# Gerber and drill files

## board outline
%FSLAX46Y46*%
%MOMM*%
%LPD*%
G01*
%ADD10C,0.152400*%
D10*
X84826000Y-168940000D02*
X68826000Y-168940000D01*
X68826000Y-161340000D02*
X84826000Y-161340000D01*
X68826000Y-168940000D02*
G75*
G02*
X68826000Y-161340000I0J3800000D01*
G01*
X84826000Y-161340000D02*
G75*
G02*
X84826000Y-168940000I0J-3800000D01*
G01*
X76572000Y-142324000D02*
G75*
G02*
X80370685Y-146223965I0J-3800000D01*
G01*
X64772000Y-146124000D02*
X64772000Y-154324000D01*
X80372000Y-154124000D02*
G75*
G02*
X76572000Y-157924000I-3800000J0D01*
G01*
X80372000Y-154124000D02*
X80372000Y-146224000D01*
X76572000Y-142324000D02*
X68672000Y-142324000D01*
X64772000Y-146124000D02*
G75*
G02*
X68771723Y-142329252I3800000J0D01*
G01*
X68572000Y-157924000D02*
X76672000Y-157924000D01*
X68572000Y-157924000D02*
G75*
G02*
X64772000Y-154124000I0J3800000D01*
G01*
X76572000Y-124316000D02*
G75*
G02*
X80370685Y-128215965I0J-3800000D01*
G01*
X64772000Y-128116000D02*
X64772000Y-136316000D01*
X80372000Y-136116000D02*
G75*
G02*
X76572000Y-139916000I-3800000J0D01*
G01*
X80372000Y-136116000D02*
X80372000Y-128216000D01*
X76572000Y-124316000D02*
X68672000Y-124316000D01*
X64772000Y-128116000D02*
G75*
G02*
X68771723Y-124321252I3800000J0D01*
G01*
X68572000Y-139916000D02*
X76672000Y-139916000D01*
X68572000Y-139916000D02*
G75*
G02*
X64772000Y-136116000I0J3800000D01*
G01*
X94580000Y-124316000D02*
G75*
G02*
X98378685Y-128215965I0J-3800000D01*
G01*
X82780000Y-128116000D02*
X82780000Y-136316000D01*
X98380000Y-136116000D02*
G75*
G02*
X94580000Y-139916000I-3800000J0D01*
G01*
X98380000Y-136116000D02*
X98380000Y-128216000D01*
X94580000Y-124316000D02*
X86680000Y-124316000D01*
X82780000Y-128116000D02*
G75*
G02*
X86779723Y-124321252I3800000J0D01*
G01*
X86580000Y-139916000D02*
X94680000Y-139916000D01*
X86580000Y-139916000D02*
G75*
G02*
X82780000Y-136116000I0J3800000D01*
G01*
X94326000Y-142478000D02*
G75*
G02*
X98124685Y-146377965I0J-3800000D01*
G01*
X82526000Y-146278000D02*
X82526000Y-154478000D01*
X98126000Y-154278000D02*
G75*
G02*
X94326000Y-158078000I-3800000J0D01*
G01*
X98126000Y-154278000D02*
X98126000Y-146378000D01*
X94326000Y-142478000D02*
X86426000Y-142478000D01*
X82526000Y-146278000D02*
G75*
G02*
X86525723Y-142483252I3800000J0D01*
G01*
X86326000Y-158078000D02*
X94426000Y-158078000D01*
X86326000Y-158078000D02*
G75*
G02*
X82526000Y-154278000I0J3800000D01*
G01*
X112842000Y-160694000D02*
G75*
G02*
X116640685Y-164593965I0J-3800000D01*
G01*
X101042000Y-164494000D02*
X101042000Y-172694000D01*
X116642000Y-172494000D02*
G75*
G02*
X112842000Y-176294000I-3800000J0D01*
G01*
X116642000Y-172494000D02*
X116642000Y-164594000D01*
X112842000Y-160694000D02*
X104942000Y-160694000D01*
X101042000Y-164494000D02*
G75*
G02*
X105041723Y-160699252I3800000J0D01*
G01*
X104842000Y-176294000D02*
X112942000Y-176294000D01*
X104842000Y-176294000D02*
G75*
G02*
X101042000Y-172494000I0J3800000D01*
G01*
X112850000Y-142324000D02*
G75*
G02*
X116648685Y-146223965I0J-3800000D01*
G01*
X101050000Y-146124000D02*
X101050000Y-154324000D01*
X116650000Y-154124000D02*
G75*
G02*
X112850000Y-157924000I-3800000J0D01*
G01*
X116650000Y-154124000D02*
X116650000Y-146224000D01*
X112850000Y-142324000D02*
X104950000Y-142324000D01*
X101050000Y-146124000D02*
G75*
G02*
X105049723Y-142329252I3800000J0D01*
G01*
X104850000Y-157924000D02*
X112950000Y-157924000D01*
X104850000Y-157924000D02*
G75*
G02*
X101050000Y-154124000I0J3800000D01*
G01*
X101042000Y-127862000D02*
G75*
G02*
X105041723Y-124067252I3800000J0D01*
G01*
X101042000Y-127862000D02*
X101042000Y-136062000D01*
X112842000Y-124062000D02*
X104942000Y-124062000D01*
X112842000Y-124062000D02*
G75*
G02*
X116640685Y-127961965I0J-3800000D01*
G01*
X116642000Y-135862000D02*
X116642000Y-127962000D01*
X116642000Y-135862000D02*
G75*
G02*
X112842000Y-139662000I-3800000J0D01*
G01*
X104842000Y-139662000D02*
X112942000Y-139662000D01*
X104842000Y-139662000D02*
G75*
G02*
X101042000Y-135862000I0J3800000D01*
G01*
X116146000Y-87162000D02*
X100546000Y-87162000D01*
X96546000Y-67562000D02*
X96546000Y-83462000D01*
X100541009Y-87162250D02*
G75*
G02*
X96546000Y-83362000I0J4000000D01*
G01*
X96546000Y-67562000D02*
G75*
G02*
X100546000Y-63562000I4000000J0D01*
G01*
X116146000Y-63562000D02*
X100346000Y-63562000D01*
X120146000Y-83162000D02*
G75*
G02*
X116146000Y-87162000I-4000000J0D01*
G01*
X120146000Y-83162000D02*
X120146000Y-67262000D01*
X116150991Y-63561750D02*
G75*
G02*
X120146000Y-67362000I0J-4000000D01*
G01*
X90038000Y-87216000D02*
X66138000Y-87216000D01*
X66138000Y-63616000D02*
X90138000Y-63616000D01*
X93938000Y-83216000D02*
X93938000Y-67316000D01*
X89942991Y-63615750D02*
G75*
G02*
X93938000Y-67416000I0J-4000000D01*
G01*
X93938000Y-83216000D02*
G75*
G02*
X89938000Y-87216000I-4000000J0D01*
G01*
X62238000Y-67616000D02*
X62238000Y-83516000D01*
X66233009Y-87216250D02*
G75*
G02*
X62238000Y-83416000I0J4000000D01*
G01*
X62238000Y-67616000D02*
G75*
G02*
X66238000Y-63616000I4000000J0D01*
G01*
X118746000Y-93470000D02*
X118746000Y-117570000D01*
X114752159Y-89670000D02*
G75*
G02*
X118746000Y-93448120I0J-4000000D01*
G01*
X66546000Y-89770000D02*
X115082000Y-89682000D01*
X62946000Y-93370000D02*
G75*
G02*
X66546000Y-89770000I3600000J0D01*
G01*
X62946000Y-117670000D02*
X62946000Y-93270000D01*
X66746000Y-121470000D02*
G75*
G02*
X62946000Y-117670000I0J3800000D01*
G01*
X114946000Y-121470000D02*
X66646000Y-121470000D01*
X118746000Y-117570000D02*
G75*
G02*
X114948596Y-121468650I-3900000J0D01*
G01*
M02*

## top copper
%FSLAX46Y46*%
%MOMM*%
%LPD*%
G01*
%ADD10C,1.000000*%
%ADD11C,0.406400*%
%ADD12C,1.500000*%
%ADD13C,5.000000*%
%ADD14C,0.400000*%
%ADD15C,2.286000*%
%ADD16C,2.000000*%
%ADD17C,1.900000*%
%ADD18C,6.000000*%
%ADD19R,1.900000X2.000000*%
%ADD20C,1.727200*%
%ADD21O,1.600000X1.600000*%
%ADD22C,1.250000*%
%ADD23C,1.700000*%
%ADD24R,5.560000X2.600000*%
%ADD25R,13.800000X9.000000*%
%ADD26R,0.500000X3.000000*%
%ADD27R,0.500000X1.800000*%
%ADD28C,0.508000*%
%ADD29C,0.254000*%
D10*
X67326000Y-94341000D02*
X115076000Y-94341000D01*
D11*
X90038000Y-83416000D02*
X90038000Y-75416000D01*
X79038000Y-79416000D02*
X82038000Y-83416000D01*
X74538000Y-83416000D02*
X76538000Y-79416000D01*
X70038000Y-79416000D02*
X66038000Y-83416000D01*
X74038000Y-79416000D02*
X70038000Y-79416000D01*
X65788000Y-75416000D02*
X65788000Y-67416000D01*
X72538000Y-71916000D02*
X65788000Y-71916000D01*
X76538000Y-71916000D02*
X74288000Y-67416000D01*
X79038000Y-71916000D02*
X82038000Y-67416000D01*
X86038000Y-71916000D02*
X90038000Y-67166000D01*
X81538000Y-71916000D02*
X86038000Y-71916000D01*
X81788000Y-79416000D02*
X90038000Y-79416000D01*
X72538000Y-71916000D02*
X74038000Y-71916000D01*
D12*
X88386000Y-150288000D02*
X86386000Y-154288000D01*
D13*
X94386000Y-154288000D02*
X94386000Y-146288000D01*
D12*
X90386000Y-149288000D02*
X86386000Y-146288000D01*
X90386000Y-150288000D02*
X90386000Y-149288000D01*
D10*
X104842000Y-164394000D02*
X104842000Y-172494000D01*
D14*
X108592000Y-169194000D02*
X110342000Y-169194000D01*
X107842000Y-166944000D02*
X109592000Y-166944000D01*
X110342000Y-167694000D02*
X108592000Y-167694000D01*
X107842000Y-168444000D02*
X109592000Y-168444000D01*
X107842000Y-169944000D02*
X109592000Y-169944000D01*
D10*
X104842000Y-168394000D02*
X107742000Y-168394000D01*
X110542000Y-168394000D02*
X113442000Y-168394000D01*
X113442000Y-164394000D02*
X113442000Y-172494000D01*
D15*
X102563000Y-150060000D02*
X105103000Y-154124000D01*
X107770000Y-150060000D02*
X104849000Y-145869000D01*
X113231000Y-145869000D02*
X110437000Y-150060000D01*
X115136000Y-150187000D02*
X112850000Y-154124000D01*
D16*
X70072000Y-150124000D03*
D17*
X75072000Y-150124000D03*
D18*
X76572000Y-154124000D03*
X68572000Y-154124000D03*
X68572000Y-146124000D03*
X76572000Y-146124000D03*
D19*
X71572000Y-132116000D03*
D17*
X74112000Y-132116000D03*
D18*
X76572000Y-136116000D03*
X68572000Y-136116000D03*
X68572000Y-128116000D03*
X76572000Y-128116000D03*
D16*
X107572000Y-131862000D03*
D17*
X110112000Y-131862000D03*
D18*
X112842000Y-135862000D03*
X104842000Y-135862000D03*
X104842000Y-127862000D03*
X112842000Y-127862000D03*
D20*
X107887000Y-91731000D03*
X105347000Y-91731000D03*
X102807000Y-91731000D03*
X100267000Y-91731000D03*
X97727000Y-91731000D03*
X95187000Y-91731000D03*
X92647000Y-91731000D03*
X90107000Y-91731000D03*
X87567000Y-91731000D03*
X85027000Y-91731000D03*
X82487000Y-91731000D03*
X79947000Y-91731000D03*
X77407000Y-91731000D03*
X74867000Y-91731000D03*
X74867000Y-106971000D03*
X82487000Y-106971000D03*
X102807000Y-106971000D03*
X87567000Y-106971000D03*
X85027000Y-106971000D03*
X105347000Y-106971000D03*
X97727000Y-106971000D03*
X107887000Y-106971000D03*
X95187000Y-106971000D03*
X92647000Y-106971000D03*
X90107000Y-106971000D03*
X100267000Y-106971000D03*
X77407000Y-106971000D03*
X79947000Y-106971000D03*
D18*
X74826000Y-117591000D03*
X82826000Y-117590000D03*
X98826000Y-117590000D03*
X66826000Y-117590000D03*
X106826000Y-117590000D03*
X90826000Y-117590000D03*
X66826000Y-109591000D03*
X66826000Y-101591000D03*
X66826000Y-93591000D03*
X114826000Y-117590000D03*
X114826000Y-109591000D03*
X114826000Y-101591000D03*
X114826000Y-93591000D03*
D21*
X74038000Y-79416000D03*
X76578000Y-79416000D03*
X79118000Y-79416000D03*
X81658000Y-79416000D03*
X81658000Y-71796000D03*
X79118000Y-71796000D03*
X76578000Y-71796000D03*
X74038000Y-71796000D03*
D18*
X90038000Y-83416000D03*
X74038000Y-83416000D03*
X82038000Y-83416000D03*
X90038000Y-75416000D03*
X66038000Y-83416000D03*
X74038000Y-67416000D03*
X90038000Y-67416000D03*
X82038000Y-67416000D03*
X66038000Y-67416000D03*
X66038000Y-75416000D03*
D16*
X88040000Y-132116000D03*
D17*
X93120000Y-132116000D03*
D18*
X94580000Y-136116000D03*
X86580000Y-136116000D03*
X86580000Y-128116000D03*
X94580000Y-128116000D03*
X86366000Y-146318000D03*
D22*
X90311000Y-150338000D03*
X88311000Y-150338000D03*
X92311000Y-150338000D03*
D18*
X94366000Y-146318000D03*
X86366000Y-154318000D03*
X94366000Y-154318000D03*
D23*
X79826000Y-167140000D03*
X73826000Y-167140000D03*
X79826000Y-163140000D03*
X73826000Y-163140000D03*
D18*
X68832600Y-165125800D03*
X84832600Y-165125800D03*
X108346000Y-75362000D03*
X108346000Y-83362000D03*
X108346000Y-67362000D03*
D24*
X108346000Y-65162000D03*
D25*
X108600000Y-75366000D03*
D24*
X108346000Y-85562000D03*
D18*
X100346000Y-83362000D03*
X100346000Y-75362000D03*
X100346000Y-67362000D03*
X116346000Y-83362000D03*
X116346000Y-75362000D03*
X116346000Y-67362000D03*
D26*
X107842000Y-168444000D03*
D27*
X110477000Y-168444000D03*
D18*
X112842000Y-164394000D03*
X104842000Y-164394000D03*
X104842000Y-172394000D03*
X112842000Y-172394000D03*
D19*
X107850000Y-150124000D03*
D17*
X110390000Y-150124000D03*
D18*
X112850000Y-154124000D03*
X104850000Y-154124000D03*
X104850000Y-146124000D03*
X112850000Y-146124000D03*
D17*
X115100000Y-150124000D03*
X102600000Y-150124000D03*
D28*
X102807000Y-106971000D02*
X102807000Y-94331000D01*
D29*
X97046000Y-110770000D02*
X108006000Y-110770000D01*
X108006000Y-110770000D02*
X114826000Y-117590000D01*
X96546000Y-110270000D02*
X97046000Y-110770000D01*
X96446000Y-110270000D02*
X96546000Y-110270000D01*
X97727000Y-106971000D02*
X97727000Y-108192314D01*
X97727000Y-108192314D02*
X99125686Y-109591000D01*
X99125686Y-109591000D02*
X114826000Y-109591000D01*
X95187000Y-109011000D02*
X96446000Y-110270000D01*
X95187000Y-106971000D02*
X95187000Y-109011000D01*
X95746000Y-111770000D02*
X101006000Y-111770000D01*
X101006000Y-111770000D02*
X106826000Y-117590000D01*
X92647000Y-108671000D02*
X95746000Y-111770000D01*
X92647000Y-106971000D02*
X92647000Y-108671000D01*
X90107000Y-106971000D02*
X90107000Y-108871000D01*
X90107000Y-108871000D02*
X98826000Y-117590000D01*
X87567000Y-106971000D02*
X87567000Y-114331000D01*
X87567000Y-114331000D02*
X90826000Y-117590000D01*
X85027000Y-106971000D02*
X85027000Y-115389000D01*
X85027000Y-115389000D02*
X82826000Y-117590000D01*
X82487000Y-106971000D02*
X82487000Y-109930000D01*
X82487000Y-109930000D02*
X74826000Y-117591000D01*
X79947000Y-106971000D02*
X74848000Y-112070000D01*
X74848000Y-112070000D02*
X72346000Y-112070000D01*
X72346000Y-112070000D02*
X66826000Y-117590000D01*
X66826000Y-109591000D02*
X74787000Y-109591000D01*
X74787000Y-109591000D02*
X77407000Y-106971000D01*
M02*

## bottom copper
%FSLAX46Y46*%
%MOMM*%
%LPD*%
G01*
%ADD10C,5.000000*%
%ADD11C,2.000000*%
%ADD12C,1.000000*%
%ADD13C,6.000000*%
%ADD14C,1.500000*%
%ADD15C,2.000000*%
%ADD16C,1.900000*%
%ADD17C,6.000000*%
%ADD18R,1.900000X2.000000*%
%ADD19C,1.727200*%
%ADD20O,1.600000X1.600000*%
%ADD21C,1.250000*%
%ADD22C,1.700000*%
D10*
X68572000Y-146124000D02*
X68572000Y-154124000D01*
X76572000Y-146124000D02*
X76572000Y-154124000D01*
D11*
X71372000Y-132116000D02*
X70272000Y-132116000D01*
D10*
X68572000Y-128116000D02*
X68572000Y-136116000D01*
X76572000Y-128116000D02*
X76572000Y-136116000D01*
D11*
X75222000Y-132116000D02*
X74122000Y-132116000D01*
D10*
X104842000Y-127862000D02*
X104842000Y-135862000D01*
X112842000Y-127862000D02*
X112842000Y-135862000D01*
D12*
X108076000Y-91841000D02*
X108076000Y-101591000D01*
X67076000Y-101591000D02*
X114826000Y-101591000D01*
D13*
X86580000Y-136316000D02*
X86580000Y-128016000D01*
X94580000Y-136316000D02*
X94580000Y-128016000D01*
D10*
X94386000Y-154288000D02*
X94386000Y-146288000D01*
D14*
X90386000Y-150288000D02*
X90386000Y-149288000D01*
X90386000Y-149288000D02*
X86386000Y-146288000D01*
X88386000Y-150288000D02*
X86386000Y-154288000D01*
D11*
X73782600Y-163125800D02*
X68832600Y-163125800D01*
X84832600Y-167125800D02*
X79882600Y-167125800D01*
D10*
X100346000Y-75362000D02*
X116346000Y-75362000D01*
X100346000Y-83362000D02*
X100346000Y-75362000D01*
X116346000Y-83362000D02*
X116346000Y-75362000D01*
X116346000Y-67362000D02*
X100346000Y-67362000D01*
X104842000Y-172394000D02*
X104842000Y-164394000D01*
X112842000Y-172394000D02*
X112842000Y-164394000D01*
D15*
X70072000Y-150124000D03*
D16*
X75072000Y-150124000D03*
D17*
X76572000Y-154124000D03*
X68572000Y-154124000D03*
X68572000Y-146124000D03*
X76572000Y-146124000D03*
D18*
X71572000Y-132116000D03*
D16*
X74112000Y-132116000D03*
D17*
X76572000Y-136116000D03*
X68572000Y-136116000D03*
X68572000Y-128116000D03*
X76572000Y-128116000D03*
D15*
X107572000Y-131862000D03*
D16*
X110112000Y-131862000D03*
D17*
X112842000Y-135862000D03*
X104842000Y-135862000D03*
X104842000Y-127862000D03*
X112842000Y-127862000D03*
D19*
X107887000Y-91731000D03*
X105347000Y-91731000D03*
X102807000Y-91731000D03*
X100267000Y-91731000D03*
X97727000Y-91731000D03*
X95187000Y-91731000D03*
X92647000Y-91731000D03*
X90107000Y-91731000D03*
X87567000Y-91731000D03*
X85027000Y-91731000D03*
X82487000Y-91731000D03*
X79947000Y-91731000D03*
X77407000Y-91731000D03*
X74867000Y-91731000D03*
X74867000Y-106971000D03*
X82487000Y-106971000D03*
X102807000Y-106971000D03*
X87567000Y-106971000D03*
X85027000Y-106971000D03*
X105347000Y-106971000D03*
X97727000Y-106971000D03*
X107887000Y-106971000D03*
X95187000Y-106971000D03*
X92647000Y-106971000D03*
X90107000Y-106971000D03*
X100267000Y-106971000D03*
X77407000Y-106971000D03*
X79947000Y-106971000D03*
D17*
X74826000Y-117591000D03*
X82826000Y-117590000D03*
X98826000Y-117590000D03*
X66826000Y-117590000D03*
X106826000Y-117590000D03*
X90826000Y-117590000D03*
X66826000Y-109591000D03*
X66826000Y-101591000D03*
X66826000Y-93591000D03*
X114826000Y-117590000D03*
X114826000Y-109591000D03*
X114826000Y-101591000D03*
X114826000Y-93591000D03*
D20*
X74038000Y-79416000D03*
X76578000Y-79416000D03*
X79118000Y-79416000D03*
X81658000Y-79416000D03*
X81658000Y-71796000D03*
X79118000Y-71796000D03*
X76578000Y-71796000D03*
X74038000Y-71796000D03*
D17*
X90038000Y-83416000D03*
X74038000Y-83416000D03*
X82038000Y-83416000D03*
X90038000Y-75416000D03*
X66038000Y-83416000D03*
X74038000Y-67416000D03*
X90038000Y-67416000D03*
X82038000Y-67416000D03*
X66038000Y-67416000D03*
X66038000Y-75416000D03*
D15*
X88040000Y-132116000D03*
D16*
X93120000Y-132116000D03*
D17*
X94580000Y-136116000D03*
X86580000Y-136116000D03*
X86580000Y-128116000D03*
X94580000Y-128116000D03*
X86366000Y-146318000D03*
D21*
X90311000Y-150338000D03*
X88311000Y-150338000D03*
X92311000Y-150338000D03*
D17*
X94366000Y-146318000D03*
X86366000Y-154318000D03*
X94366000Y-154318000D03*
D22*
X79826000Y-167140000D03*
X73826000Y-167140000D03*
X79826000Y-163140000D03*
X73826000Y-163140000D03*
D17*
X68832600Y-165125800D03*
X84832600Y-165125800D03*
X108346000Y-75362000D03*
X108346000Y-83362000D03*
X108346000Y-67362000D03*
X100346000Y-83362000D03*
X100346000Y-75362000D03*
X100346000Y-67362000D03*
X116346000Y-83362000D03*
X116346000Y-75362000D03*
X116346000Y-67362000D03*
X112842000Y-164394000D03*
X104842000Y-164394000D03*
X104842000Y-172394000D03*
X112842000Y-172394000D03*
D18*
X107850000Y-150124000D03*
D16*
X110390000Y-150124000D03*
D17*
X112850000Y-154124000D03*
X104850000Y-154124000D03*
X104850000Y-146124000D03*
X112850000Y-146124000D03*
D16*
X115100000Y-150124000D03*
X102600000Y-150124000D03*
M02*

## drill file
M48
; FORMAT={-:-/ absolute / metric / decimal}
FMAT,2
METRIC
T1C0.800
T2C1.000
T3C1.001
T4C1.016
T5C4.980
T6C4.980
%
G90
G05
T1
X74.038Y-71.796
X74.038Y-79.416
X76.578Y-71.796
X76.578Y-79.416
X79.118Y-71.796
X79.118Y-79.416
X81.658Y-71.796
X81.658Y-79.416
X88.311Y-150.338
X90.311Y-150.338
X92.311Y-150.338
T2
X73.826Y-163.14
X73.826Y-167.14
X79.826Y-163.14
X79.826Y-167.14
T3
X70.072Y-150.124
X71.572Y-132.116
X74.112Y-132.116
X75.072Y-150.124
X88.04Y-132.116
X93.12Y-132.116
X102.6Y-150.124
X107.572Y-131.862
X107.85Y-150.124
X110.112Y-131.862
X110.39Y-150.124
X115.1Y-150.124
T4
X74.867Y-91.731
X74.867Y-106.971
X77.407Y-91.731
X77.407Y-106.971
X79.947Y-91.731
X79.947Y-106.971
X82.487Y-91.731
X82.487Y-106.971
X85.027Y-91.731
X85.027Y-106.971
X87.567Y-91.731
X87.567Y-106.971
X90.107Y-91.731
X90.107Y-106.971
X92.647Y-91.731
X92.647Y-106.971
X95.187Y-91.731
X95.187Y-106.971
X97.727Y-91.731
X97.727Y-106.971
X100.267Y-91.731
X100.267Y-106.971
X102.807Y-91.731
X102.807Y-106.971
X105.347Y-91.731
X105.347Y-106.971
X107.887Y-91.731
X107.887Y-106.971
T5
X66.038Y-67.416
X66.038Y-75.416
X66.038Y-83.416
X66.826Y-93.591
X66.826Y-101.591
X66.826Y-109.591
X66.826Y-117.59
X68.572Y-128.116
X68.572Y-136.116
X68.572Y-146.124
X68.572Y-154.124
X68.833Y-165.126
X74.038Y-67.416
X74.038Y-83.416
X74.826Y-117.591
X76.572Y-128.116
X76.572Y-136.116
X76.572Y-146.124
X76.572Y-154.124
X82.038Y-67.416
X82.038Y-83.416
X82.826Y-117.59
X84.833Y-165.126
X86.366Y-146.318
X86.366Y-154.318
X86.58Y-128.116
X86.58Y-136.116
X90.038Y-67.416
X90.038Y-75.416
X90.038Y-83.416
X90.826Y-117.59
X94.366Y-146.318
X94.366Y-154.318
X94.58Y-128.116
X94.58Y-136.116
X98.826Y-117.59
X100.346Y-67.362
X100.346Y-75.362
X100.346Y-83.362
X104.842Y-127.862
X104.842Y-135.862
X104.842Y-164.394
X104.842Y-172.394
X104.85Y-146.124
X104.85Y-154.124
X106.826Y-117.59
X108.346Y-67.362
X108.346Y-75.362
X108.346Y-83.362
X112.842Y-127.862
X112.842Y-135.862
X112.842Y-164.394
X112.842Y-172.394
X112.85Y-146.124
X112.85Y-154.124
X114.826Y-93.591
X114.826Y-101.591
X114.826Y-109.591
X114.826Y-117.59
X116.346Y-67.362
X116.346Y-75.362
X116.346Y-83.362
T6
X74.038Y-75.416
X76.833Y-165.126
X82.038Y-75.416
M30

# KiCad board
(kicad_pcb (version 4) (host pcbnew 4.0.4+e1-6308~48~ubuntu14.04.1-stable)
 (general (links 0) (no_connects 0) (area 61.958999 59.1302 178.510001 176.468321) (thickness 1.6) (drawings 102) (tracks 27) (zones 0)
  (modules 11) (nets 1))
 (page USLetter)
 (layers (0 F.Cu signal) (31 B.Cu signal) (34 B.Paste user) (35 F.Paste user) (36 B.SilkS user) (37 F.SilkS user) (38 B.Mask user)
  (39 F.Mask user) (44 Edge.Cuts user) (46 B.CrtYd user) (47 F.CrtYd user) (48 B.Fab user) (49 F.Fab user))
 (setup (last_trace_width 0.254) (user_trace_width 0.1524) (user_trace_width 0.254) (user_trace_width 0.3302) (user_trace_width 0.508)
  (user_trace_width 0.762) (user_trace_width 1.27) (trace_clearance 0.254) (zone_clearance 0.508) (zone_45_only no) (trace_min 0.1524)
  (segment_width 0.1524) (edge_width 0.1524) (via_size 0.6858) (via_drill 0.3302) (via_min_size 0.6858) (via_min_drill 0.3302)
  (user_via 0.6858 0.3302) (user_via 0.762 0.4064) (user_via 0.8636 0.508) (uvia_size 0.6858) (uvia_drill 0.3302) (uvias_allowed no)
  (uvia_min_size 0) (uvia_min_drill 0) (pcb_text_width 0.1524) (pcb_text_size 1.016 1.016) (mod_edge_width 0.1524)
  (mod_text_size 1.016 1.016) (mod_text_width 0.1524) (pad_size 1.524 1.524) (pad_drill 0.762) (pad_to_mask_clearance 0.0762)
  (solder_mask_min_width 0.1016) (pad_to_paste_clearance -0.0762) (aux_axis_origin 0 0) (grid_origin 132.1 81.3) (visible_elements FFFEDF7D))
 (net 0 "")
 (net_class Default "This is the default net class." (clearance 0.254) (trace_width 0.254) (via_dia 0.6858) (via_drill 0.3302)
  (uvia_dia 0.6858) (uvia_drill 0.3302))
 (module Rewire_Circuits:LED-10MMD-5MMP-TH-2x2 (layer F.Cu) (at 76.572 154.124 90)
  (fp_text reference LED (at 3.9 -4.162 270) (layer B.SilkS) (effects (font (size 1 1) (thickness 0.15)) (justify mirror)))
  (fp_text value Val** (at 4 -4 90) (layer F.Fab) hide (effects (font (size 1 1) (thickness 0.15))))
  (fp_line (start 8 -8) (end 0 -8) (layer B.Cu) (width 5)) (fp_line (start 8 0) (end 0 0) (layer B.Cu) (width 5))
  (pad + thru_hole circle (at 4 -6.5 90) (size 2 2) (drill 1.00076) (layers *.Cu *.Mask F.SilkS))
  (pad - thru_hole circle (at 4 -1.5) (size 1.9 1.9) (drill 1.00076) (layers *.Cu *.Mask F.SilkS))
  (pad - thru_hole circle (at 0 0 90) (size 6 6) (drill 4.98) (layers *.Cu *.Mask))
  (pad + thru_hole circle (at 0 -8 90) (size 6 6) (drill 4.98) (layers *.Cu *.Mask))
  (pad + thru_hole circle (at 8 -8 90) (size 6 6) (drill 4.98) (layers *.Cu *.Mask))
  (pad - thru_hole circle (at 8 0 90) (size 6 6) (drill 4.98) (layers *.Cu *.Mask)))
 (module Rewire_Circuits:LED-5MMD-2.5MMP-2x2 (layer F.Cu) (at 76.572 136.116 90)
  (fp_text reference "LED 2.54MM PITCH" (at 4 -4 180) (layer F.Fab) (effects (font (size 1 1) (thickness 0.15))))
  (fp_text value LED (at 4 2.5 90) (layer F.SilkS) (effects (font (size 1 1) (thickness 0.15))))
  (fp_line (start 4 -5.2) (end 4 -6.3) (layer B.Cu) (width 2)) (fp_line (start 8 -8) (end 0 -8) (layer B.Cu) (width 5))
  (fp_line (start 8 0) (end 0 0) (layer B.Cu) (width 5))
  (fp_line (start 4 -1.35) (end 4 -2.45) (layer B.Cu) (width 2))
  (pad - thru_hole rect (at 4 -5 90) (size 2 1.9) (drill 1.00076) (layers *.Cu *.Mask))
  (pad + thru_hole circle (at 4 -2.46) (size 1.9 1.9) (drill 1.00076) (layers *.Cu *.Mask))
  (pad + thru_hole circle (at 0 0 90) (size 6 6) (drill 4.98) (layers *.Cu *.Mask))
  (pad - thru_hole circle (at 0 -8 90) (size 6 6) (drill 4.98) (layers *.Cu *.Mask))
  (pad - thru_hole circle (at 8 -8 90) (size 6 6) (drill 4.98) (layers *.Cu *.Mask))
  (pad + thru_hole circle (at 8 0 90) (size 6 6) (drill 4.98) (layers *.Cu *.Mask)))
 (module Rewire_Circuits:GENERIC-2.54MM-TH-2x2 (layer F.Cu) (at 112.842 135.862 90)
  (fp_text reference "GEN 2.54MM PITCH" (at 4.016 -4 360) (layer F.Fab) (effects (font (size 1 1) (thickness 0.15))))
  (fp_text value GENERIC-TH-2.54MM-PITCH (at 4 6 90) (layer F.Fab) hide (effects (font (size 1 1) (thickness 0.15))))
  (fp_line (start 8 -8) (end 0 -8) (layer B.Cu) (width 5)) (fp_line (start 8 0) (end 0 0) (layer B.Cu) (width 5))
  (pad 1 thru_hole circle (at 4 -5.27 90) (size 2 2) (drill 1.00076) (layers *.Cu *.Mask F.SilkS))
  (pad 2 thru_hole circle (at 4 -2.73) (size 1.9 1.9) (drill 1.00076) (layers *.Cu *.Mask F.SilkS))
  (pad 2 thru_hole circle (at 0 0 90) (size 6 6) (drill 4.98) (layers *.Cu *.Mask))
  (pad 1 thru_hole circle (at 0 -8 90) (size 6 6) (drill 4.98) (layers *.Cu *.Mask))
  (pad 1 thru_hole circle (at 8 -8 90) (size 6 6) (drill 4.98) (layers *.Cu *.Mask))
  (pad 2 thru_hole circle (at 8 0 90) (size 6 6) (drill 4.98) (layers *.Cu *.Mask)))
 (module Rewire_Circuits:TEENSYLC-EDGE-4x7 (layer F.Cu) (at 66.826 117.591 90)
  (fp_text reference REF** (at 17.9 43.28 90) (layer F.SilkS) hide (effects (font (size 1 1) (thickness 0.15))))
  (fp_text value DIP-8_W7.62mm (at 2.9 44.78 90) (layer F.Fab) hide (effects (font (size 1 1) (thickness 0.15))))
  (fp_line (start 25.75 41.25) (end 16 41.25) (layer B.Cu) (width 1)) (fp_line (start 16 0.25) (end 16 48) (layer B.Cu) (width 1))
  (fp_line (start 23.25 0.5) (end 23.25 48.25) (layer F.Cu) (width 1))
  (pad GND thru_hole circle (at 25.86 41.061 270) (size 1.7272 1.7272) (drill 1.016) (layers *.Cu *.Mask F.SilkS))
  (pad 0 thru_hole circle (at 25.86 38.521 270) (size 1.7272 1.7272) (drill 1.016) (layers *.Cu *.Mask F.SilkS))
  (pad 1 thru_hole circle (at 25.86 35.981 270) (size 1.7272 1.7272) (drill 1.016) (layers *.Cu *.Mask F.SilkS))
  (pad 2 thru_hole circle (at 25.86 33.441 270) (size 1.7272 1.7272) (drill 1.016) (layers *.Cu *.Mask F.SilkS))
  (pad 3 thru_hole circle (at 25.86 30.901 270) (size 1.7272 1.7272) (drill 1.016) (layers *.Cu *.Mask F.SilkS))
  (pad 4 thru_hole circle (at 25.86 28.361 270) (size 1.7272 1.7272) (drill 1.016) (layers *.Cu *.Mask F.SilkS))
  (pad 5 thru_hole circle (at 25.86 25.821 270) (size 1.7272 1.7272) (drill 1.016) (layers *.Cu *.Mask F.SilkS))
  (pad 6 thru_hole circle (at 25.86 23.281 270) (size 1.7272 1.7272) (drill 1.016) (layers *.Cu *.Mask F.SilkS))
  (pad 7 thru_hole circle (at 25.86 20.741 270) (size 1.7272 1.7272) (drill 1.016) (layers *.Cu *.Mask F.SilkS))
  (pad 8 thru_hole circle (at 25.86 18.201 270) (size 1.7272 1.7272) (drill 1.016) (layers *.Cu *.Mask F.SilkS))
  (pad 9 thru_hole circle (at 25.86 15.661 270) (size 1.7272 1.7272) (drill 1.016) (layers *.Cu *.Mask F.SilkS))
  (pad 10 thru_hole circle (at 25.86 13.121 270) (size 1.7272 1.7272) (drill 1.016) (layers *.Cu *.Mask F.SilkS))
  (pad 11 thru_hole circle (at 25.86 10.581 270) (size 1.7272 1.7272) (drill 1.016) (layers *.Cu *.Mask F.SilkS))
  (pad 12 thru_hole circle (at 25.86 8.041 270) (size 1.7272 1.7272) (drill 1.016) (layers *.Cu *.Mask F.SilkS))
  (pad 13 thru_hole circle (at 10.62 8.041 270) (size 1.7272 1.7272) (drill 1.016) (layers *.Cu *.Mask F.SilkS))
  (pad 16 thru_hole circle (at 10.62 15.661 270) (size 1.7272 1.7272) (drill 1.016) (layers *.Cu *.Mask F.SilkS))
  (pad 3.3V thru_hole circle (at 10.62 35.981 270) (size 1.7272 1.7272) (drill 1.016) (layers *.Cu *.Mask F.SilkS))
  (pad 18 thru_hole circle (at 10.62 20.741 270) (size 1.7272 1.7272) (drill 1.016) (layers *.Cu *.Mask F.SilkS))
  (pad 17 thru_hole circle (at 10.62 18.201 270) (size 1.7272 1.7272) (drill 1.016) (layers *.Cu *.Mask F.SilkS))
  (pad G3 thru_hole circle (at 10.62 38.521 270) (size 1.7272 1.7272) (drill 1.016) (layers *.Cu *.Mask F.SilkS))
  (pad 22 thru_hole circle (at 10.62 30.901 270) (size 1.7272 1.7272) (drill 1.016) (layers *.Cu *.Mask F.SilkS))
  (pad VIN thru_hole circle (at 10.62 41.061 270) (size 1.7272 1.7272) (drill 1.016) (layers *.Cu *.Mask F.SilkS))
  (pad 21 thru_hole circle (at 10.62 28.361 270) (size 1.7272 1.7272) (drill 1.016) (layers *.Cu *.Mask F.SilkS))
  (pad 20 thru_hole circle (at 10.62 25.821 270) (size 1.7272 1.7272) (drill 1.016) (layers *.Cu *.Mask F.SilkS))
  (pad 19 thru_hole circle (at 10.62 23.281 270) (size 1.7272 1.7272) (drill 1.016) (layers *.Cu *.Mask F.SilkS))
  (pad 23 thru_hole circle (at 10.62 33.441 270) (size 1.7272 1.7272) (drill 1.016) (layers *.Cu *.Mask F.SilkS))
  (pad 14 thru_hole circle (at 10.62 10.581 270) (size 1.7272 1.7272) (drill 1.016) (layers *.Cu *.Mask F.SilkS))
  (pad 15 thru_hole circle (at 10.62 13.121 270) (size 1.7272 1.7272) (drill 1.016) (layers *.Cu *.Mask F.SilkS))
  (pad 16 thru_hole circle (at 0 8 180) (size 6 6) (drill 4.98) (layers *.Cu *.Mask))
  (pad 17 thru_hole circle (at 0.001 16 180) (size 6 6) (drill 4.98) (layers *.Cu *.Mask))
  (pad 19 thru_hole circle (at 0.001 32 180) (size 6 6) (drill 4.98) (layers *.Cu *.Mask))
  (pad 15 thru_hole circle (at 0.001 0 180) (size 6 6) (drill 4.98) (layers *.Cu *.Mask))
  (pad 20 thru_hole circle (at 0.001 40 180) (size 6 6) (drill 4.98) (layers *.Cu *.Mask))
  (pad 18 thru_hole circle (at 0.001 24 180) (size 6 6) (drill 4.98) (layers *.Cu *.Mask))
  (pad 14 thru_hole circle (at 8 0 180) (size 6 6) (drill 4.98) (layers *.Cu *.Mask))
  (pad GND thru_hole circle (at 16 0 180) (size 6 6) (drill 4.98) (layers *.Cu *.Mask))
  (pad 3.3V thru_hole circle (at 24 0 180) (size 6 6) (drill 4.98) (layers *.Cu *.Mask))
  (pad 21 thru_hole circle (at 0.001 48 180) (size 6 6) (drill 4.98) (layers *.Cu *.Mask))
  (pad 22 thru_hole circle (at 8 48 180) (size 6 6) (drill 4.98) (layers *.Cu *.Mask))
  (pad GND thru_hole circle (at 16 48 180) (size 6 6) (drill 4.98) (layers *.Cu *.Mask))
  (pad 3.3V thru_hole circle (at 24 48 180) (size 6 6) (drill 4.98) (layers *.Cu *.Mask)))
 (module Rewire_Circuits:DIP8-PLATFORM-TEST (layer F.Cu) (at 90.038 83.416 90)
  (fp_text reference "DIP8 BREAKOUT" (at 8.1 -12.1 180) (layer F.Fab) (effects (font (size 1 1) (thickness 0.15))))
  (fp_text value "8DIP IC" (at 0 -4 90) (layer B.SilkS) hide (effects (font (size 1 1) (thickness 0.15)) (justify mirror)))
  (fp_line (start 0 0) (end 8 0) (layer F.Cu) (width 0.4064))
  (fp_line (start 4 -11) (end 0 -8) (layer F.Cu) (width 0.4064))
  (fp_line (start 0 -15.5) (end 4 -13.5) (layer F.Cu) (width 0.4064))
  (fp_line (start 4 -20) (end 0 -24) (layer F.Cu) (width 0.4064))
  (fp_line (start 4 -16) (end 4 -20) (layer F.Cu) (width 0.4064))
  (fp_line (start 8 -24.25) (end 16 -24.25) (layer F.Cu) (width 0.4064))
  (fp_line (start 11.5 -17.5) (end 11.5 -24.25) (layer F.Cu) (width 0.4064))
  (fp_line (start 11.5 -13.5) (end 16 -15.75) (layer F.Cu) (width 0.4064))
  (fp_line (start 11.5 -11) (end 16 -8) (layer F.Cu) (width 0.4064))
  (fp_line (start 11.5 -4) (end 16.25 0) (layer F.Cu) (width 0.4064))
  (fp_line (start 11.5 -8.5) (end 11.5 -4) (layer F.Cu) (width 0.4064))
  (fp_line (start 4 -8.25) (end 4 0) (layer F.Cu) (width 0.4064))
  (fp_line (start 11.5 -17.5) (end 11.5 -16) (layer F.Cu) (width 0.4064))
  (pad 1 thru_hole oval (at 4 -16 90) (size 1.6 1.6) (drill 0.8) (layers *.Cu *.Mask F.SilkS))
  (pad 2 thru_hole oval (at 4 -13.46 90) (size 1.6 1.6) (drill 0.8) (layers *.Cu *.Mask F.SilkS))
  (pad 3 thru_hole oval (at 4 -10.92 90) (size 1.6 1.6) (drill 0.8) (layers *.Cu *.Mask F.SilkS))
  (pad 4 thru_hole oval (at 4 -8.38 90) (size 1.6 1.6) (drill 0.8) (layers *.Cu *.Mask F.SilkS))
  (pad 5 thru_hole oval (at 11.62 -8.38 90) (size 1.6 1.6) (drill 0.8) (layers *.Cu *.Mask F.SilkS))
  (pad 6 thru_hole oval (at 11.62 -10.92 90) (size 1.6 1.6) (drill 0.8) (layers *.Cu *.Mask F.SilkS))
  (pad 7 thru_hole oval (at 11.62 -13.46 90) (size 1.6 1.6) (drill 0.8) (layers *.Cu *.Mask F.SilkS))
  (pad 8 thru_hole oval (at 11.62 -16 90) (size 1.6 1.6) (drill 0.8) (layers *.Cu *.Mask F.SilkS))
  (pad 4 thru_hole circle (at 0 0) (size 6 6) (drill 4.98) (layers *.Cu *.Mask))
  (pad "" np_thru_hole circle (at 8 -16) (size 4.88 4.88) (drill 4.98) (layers *.Cu *.Mask))
  (pad 2 thru_hole circle (at 0 -16) (size 6 6) (drill 4.98) (layers *.Cu *.Mask))
  (pad 3 thru_hole circle (at 0 -8) (size 6 6) (drill 4.98) (layers *.Cu *.Mask))
  (pad "" np_thru_hole circle (at 8 -8) (size 4.88 4.88) (drill 4.98) (layers *.Cu *.Mask F.SilkS))
  (pad 4 thru_hole circle (at 8 0) (size 6 6) (drill 4.98) (layers *.Cu *.Mask))
  (pad 1 thru_hole circle (at 0 -24) (size 6 6) (drill 4.98) (layers *.Cu *.Mask))
  (pad 7 thru_hole circle (at 16 -16) (size 6 6) (drill 4.98) (layers *.Cu *.Mask))
  (pad 5 thru_hole circle (at 16 0) (size 6 6) (drill 4.98) (layers *.Cu *.Mask))
  (pad 6 thru_hole circle (at 16 -8) (size 6 6) (drill 4.98) (layers *.Cu *.Mask))
  (pad 8 thru_hole circle (at 16 -24) (size 6 6) (drill 4.98) (layers *.Cu *.Mask))
  (pad 8 thru_hole circle (at 8 -24) (size 6 6) (drill 4.98) (layers *.Cu *.Mask)))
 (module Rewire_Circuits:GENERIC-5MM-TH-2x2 (layer F.Cu) (at 94.58 136.116 90)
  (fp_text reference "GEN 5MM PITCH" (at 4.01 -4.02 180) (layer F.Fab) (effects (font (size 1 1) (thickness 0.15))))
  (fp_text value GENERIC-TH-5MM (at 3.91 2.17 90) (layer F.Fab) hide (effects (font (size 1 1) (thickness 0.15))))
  (fp_line (start -0.2 -8) (end 8.1 -8) (layer B.Cu) (width 6)) (fp_line (start -0.2 0) (end 8.1 0) (layer B.Cu) (width 6))
  (pad 1 thru_hole circle (at 4 -6.54 90) (size 2 2) (drill 1.00076) (layers *.Cu *.Mask F.SilkS))
  (pad 2 thru_hole circle (at 4 -1.46) (size 1.9 1.9) (drill 1.00076) (layers *.Cu *.Mask F.SilkS))
  (pad 2 thru_hole circle (at 0 0 90) (size 6 6) (drill 4.98) (layers *.Cu *.Mask))
  (pad 1 thru_hole circle (at 0 -8 90) (size 6 6) (drill 4.98) (layers *.Cu *.Mask))
  (pad 1 thru_hole circle (at 8 -8 90) (size 6 6) (drill 4.98) (layers *.Cu *.Mask))
  (pad 2 thru_hole circle (at 8 0 90) (size 6 6) (drill 4.98) (layers *.Cu *.Mask)))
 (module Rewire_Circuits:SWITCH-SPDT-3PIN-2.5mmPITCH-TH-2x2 (layer F.Cu) (at 94.366 154.318 90)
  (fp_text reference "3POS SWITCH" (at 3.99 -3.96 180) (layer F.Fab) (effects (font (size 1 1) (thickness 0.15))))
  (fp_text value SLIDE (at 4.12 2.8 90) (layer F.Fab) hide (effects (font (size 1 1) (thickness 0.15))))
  (fp_line (start 4.03 -5.98) (end 0.03 -7.98) (layer F.Cu) (width 1.5))
  (fp_line (start 0.03 0.02) (end 8.03 0.02) (layer B.Cu) (width 5))
  (fp_line (start 4.03 -3.98) (end 5.03 -3.98) (layer B.Cu) (width 1.5))
  (fp_line (start 5.03 -3.98) (end 8.03 -7.98) (layer B.Cu) (width 1.5))
  (fp_line (start 0.03 0.02) (end 8.03 0.02) (layer F.Cu) (width 5))
  (fp_line (start 5.03 -3.98) (end 8.03 -7.98) (layer F.Cu) (width 1.5))
  (fp_line (start 4.03 -3.98) (end 5.03 -3.98) (layer F.Cu) (width 1.5))
  (fp_line (start 4.03 -5.98) (end 0.03 -7.98) (layer B.Cu) (width 1.5))
  (pad 2 thru_hole circle (at 8 -8 90) (size 6 6) (drill 4.98) (layers *.Cu *.Mask))
  (pad 2 thru_hole circle (at 3.98 -4.055) (size 1.25 1.25) (drill 0.8) (layers *.Cu *.Mask))
  (pad 3 thru_hole circle (at 3.98 -6.055) (size 1.25 1.25) (drill 0.8) (layers *.Cu *.Mask))
  (pad 1 thru_hole circle (at 3.98 -2.055) (size 1.25 1.25) (drill 0.8) (layers *.Cu *.Mask))
  (pad 1 thru_hole circle (at 8 0 90) (size 6 6) (drill 4.98) (layers *.Cu *.Mask))
  (pad 3 thru_hole circle (at 0 -8 90) (size 6 6) (drill 4.98) (layers *.Cu *.Mask))
  (pad 1 thru_hole circle (at 0 0 90) (size 6 6) (drill 4.98) (layers *.Cu *.Mask)))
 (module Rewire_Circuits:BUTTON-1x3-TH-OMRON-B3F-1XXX (layer F.Cu) (at 68.8326 165.1258)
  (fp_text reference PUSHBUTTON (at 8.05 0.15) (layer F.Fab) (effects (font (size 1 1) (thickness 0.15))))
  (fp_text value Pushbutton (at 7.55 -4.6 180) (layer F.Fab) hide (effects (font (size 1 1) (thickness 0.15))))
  (fp_line (start 4.95 -2) (end 0 -2) (layer B.Cu) (width 2)) (fp_line (start 16 2) (end 11.05 2) (layer B.Cu) (width 2))
  (pad 2 thru_hole circle (at 10.9934 2.0142) (size 1.7 1.7) (drill 1) (layers *.Cu *.Mask))
  (pad 2 thru_hole circle (at 4.9934 2.0142) (size 1.7 1.7) (drill 1) (layers *.Cu *.Mask))
  (pad 1 thru_hole circle (at 10.9934 -1.9858) (size 1.7 1.7) (drill 1) (layers *.Cu *.Mask))
  (pad 1 thru_hole circle (at 4.9934 -1.9858) (size 1.7 1.7) (drill 1) (layers *.Cu *.Mask))
  (pad "" np_thru_hole circle (at 8 0) (size 4.88 4.88) (drill 4.98) (layers *.Cu *.Mask F.SilkS))
  (pad 1 thru_hole circle (at 0 0) (size 6 6) (drill 4.98) (layers *.Cu *.Mask F.SilkS))
  (pad 2 thru_hole circle (at 16 0) (size 6 6) (drill 4.98) (layers *.Cu *.Mask F.SilkS)))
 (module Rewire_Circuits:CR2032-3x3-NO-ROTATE (layer F.Cu) (at 116.346 83.362 90)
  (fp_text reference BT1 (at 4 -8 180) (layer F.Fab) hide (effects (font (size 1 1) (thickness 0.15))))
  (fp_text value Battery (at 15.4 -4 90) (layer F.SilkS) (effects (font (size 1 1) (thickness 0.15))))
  (fp_line (start 8 -16) (end 8 0) (layer B.Cu) (width 5)) (fp_line (start 0 -16) (end 8 -16) (layer B.Cu) (width 5))
  (fp_line (start 0 0) (end 8 0) (layer B.Cu) (width 5)) (fp_line (start 16 0) (end 16 -16) (layer B.Cu) (width 5))
  (pad GND thru_hole circle (at 8 -8 90) (size 6 6) (drill 4.98) (layers *.Cu *.Mask))
  (pad + thru_hole circle (at 0 -8 90) (size 6 6) (drill 4.98) (layers *.Cu *.Mask))
  (pad + thru_hole circle (at 16 -8 90) (size 6 6) (drill 4.98) (layers *.Cu *.Mask))
  (pad + smd rect (at 18.2 -8 90) (size 2.6 5.56) (layers F.Cu F.Paste F.Mask))
  (pad GND smd rect (at 7.996 -7.746 90) (size 9 13.8) (layers F.Cu F.Paste F.Mask))
  (pad + smd rect (at -2.2 -8 90) (size 2.6 5.56) (layers F.Cu F.Paste F.Mask))
  (pad GND thru_hole circle (at 0 -16 90) (size 6 6) (drill 4.98) (layers *.Cu *.Mask))
  (pad GND thru_hole circle (at 8 -16 90) (size 6 6) (drill 4.98) (layers *.Cu *.Mask))
  (pad + thru_hole circle (at 16 -16 90) (size 6 6) (drill 4.98) (layers *.Cu B.Mask))
  (pad GND thru_hole circle (at 0 0 90) (size 6 6) (drill 4.98) (layers *.Cu *.Mask))
  (pad GND thru_hole circle (at 8 0 90) (size 6 6) (drill 4.98) (layers *.Cu *.Mask))
  (pad + thru_hole circle (at 16 0 90) (size 6 6) (drill 4.98) (layers *.Cu B.Mask)))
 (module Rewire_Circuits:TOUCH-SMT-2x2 (layer F.Cu) (at 112.842 172.394 90)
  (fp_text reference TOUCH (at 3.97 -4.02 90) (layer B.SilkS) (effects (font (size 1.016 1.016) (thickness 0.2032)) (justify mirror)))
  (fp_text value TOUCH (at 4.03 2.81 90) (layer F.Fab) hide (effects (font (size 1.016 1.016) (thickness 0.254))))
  (fp_line (start 0 -8) (end 8 -8) (layer B.Cu) (width 5)) (fp_line (start 8 -8) (end -0.1 -8) (layer F.Cu) (width 1))
  (fp_line (start 3.2 -4.25) (end 3.2 -2.5) (layer F.Cu) (width 0.4))
  (fp_line (start 5.45 -5) (end 5.45 -3.25) (layer F.Cu) (width 0.4))
  (fp_line (start 4.7 -2.5) (end 4.7 -4.25) (layer F.Cu) (width 0.4))
  (fp_line (start 3.95 -5) (end 3.95 -3.25) (layer F.Cu) (width 0.4))
  (fp_line (start 2.45 -5) (end 2.45 -3.25) (layer F.Cu) (width 0.4)) (fp_line (start 4 -8) (end 4 -5.1) (layer F.Cu) (width 1))
  (fp_line (start 4 -2.3) (end 4 0.6) (layer F.Cu) (width 1))
  (fp_line (start 8 0.6) (end -0.1 0.6) (layer F.Cu) (width 1)) (fp_line (start 0 0) (end 8 0) (layer B.Cu) (width 5))
  (pad 1 smd rect (at 3.95 -5 90) (size 3 0.5) (layers F.Cu F.Paste F.Mask))
  (pad 2 smd rect (at 3.95 -2.365 90) (size 1.8 0.5) (layers F.Cu F.Paste F.Mask))
  (pad 3 smd circle (at 3.95 -4 90) (size 4 4) (layers F.Paste F.Mask))
  (pad 2 thru_hole circle (at 8 0 90) (size 6 6) (drill 4.98) (layers *.Cu *.Mask))
  (pad 1 thru_hole circle (at 8 -8 90) (size 6 6) (drill 4.98) (layers *.Cu *.Mask))
  (pad 1 thru_hole circle (at 0 -8 90) (size 6 6) (drill 4.98) (layers *.Cu *.Mask))
  (pad 2 thru_hole circle (at 0 0 90) (size 6 6) (drill 4.98) (layers *.Cu *.Mask)))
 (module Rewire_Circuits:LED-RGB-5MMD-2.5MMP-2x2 (layer F.Cu) (at 112.85 154.124 90)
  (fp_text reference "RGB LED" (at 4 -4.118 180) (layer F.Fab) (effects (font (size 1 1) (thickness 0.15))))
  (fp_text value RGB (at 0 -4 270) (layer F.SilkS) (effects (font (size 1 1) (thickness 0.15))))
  (fp_line (start 4.064 -10.287) (end 0 -7.747) (layer F.Cu) (width 2.286))
  (fp_line (start 4.064 -5.08) (end 8.255 -8.001) (layer F.Cu) (width 2.286))
  (fp_line (start 8.255 0.381) (end 4.064 -2.413) (layer F.Cu) (width 2.286))
  (fp_line (start 3.937 2.286) (end 0 0) (layer F.Cu) (width 2.286))
  (pad 2 thru_hole rect (at 4 -5 90) (size 2 1.9) (drill 1.00076) (layers *.Cu *.Mask))
  (pad 3 thru_hole circle (at 4 -2.46) (size 1.9 1.9) (drill 1.00076) (layers *.Cu *.Mask))
  (pad 4 thru_hole circle (at 0 0 90) (size 6 6) (drill 4.98) (layers *.Cu *.Mask))
  (pad 1 thru_hole circle (at 0 -8 90) (size 6 6) (drill 4.98) (layers *.Cu *.Mask))
  (pad 2 thru_hole circle (at 8 -8 90) (size 6 6) (drill 4.98) (layers *.Cu *.Mask))
  (pad 3 thru_hole circle (at 8 0 90) (size 6 6) (drill 4.98) (layers *.Cu *.Mask))
  (pad 4 thru_hole circle (at 4 2.25) (size 1.9 1.9) (drill 1.00076) (layers *.Cu *.Mask))
  (pad 1 thru_hole circle (at 4 -10.25) (size 1.9 1.9) (drill 1.00076) (layers *.Cu *.Mask)))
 (gr_line (start 84.826 168.94) (end 68.826 168.94) (layer Edge.Cuts) (width 0.1524))
 (gr_line (start 68.826 161.34) (end 84.826 161.34) (layer Edge.Cuts) (width 0.1524))
 (gr_arc (start 68.826 165.14) (end 68.826 168.94) (angle 180) (layer Edge.Cuts) (width 0.1524))
 (gr_arc (start 84.826 165.14) (end 84.826 161.34) (angle 180) (layer Edge.Cuts) (width 0.1524))
 (gr_arc (start 76.572 146.124) (end 76.572 142.324) (angle 91.50743021) (layer Edge.Cuts) (width 0.1524))
 (gr_line (start 64.772 146.124) (end 64.772 154.324) (layer Edge.Cuts) (width 0.1524))
 (gr_arc (start 76.572 154.124) (end 80.372 154.124) (angle 90) (layer Edge.Cuts) (width 0.1524))
 (gr_line (start 80.372 154.124) (end 80.372 146.224) (layer Edge.Cuts) (width 0.1524))
 (gr_line (start 76.572 142.324) (end 68.672 142.324) (layer Edge.Cuts) (width 0.1524))
 (gr_arc (start 68.572 146.124) (end 64.772 146.124) (angle 93.01277958) (layer Edge.Cuts) (width 0.1524))
 (gr_line (start 68.572 157.924) (end 76.672 157.924) (layer Edge.Cuts) (width 0.1524))
 (gr_arc (start 68.572 154.124) (end 68.572 157.924) (angle 90) (layer Edge.Cuts) (width 0.1524))
 (gr_arc (start 76.572 128.116) (end 76.572 124.316) (angle 91.50743021) (layer Edge.Cuts) (width 0.1524))
 (gr_line (start 64.772 128.116) (end 64.772 136.316) (layer Edge.Cuts) (width 0.1524))
 (gr_arc (start 76.572 136.116) (end 80.372 136.116) (angle 90) (layer Edge.Cuts) (width 0.1524))
 (gr_line (start 80.372 136.116) (end 80.372 128.216) (layer Edge.Cuts) (width 0.1524))
 (gr_line (start 76.572 124.316) (end 68.672 124.316) (layer Edge.Cuts) (width 0.1524))
 (gr_arc (start 68.572 128.116) (end 64.772 128.116) (angle 93.01277958) (layer Edge.Cuts) (width 0.1524))
 (gr_line (start 68.572 139.916) (end 76.672 139.916) (layer Edge.Cuts) (width 0.1524))
 (gr_arc (start 68.572 136.116) (end 68.572 139.916) (angle 90) (layer Edge.Cuts) (width 0.1524))
 (gr_arc (start 94.58 128.116) (end 94.58 124.316) (angle 91.50743021) (layer Edge.Cuts) (width 0.1524))
 (gr_line (start 82.78 128.116) (end 82.78 136.316) (layer Edge.Cuts) (width 0.1524))
 (gr_arc (start 94.58 136.116) (end 98.38 136.116) (angle 90) (layer Edge.Cuts) (width 0.1524))
 (gr_line (start 98.38 136.116) (end 98.38 128.216) (layer Edge.Cuts) (width 0.1524))
 (gr_line (start 94.58 124.316) (end 86.68 124.316) (layer Edge.Cuts) (width 0.1524))
 (gr_arc (start 86.58 128.116) (end 82.78 128.116) (angle 93.01277958) (layer Edge.Cuts) (width 0.1524))
 (gr_line (start 86.58 139.916) (end 94.68 139.916) (layer Edge.Cuts) (width 0.1524))
 (gr_arc (start 86.58 136.116) (end 86.58 139.916) (angle 90) (layer Edge.Cuts) (width 0.1524))
 (gr_arc (start 94.326 146.278) (end 94.326 142.478) (angle 91.50743021) (layer Edge.Cuts) (width 0.1524))
 (gr_line (start 82.526 146.278) (end 82.526 154.478) (layer Edge.Cuts) (width 0.1524))
 (gr_arc (start 94.326 154.278) (end 98.126 154.278) (angle 90) (layer Edge.Cuts) (width 0.1524))
 (gr_line (start 98.126 154.278) (end 98.126 146.378) (layer Edge.Cuts) (width 0.1524))
 (gr_line (start 94.326 142.478) (end 86.426 142.478) (layer Edge.Cuts) (width 0.1524))
 (gr_arc (start 86.326 146.278) (end 82.526 146.278) (angle 93.01277958) (layer Edge.Cuts) (width 0.1524))
 (gr_line (start 86.326 158.078) (end 94.426 158.078) (layer Edge.Cuts) (width 0.1524))
 (gr_arc (start 86.326 154.278) (end 86.326 158.078) (angle 90) (layer Edge.Cuts) (width 0.1524))
 (gr_arc (start 112.842 164.494) (end 112.842 160.694) (angle 91.50743021) (layer Edge.Cuts) (width 0.1524))
 (gr_line (start 101.042 164.494) (end 101.042 172.694) (layer Edge.Cuts) (width 0.1524))
 (gr_arc (start 112.842 172.494) (end 116.642 172.494) (angle 90) (layer Edge.Cuts) (width 0.1524))
 (gr_line (start 116.642 172.494) (end 116.642 164.594) (layer Edge.Cuts) (width 0.1524))
 (gr_line (start 112.842 160.694) (end 104.942 160.694) (layer Edge.Cuts) (width 0.1524))
 (gr_arc (start 104.842 164.494) (end 101.042 164.494) (angle 93.01277958) (layer Edge.Cuts) (width 0.1524))
 (gr_line (start 104.842 176.294) (end 112.942 176.294) (layer Edge.Cuts) (width 0.1524))
 (gr_arc (start 104.842 172.494) (end 104.842 176.294) (angle 90) (layer Edge.Cuts) (width 0.1524))
 (gr_arc (start 112.85 146.124) (end 112.85 142.324) (angle 91.50743021) (layer Edge.Cuts) (width 0.1524))
 (gr_line (start 101.05 146.124) (end 101.05 154.324) (layer Edge.Cuts) (width 0.1524))
 (gr_arc (start 112.85 154.124) (end 116.65 154.124) (angle 90) (layer Edge.Cuts) (width 0.1524))
 (gr_line (start 116.65 154.124) (end 116.65 146.224) (layer Edge.Cuts) (width 0.1524))
 (gr_line (start 112.85 142.324) (end 104.95 142.324) (layer Edge.Cuts) (width 0.1524))
 (gr_arc (start 104.85 146.124) (end 101.05 146.124) (angle 93.01277958) (layer Edge.Cuts) (width 0.1524))
 (gr_line (start 104.85 157.924) (end 112.95 157.924) (layer Edge.Cuts) (width 0.1524))
 (gr_arc (start 104.85 154.124) (end 104.85 157.924) (angle 90) (layer Edge.Cuts) (width 0.1524))
 (gr_arc (start 104.842 127.862) (end 101.042 127.862) (angle 93.01277958) (layer Edge.Cuts) (width 0.1524))
 (gr_line (start 101.042 127.862) (end 101.042 136.062) (layer Edge.Cuts) (width 0.1524))
 (gr_line (start 112.842 124.062) (end 104.942 124.062) (layer Edge.Cuts) (width 0.1524))
 (gr_arc (start 112.842 127.862) (end 112.842 124.062) (angle 91.50743021) (layer Edge.Cuts) (width 0.1524))
 (gr_line (start 116.642 135.862) (end 116.642 127.962) (layer Edge.Cuts) (width 0.1524))
 (gr_arc (start 112.842 135.862) (end 116.642 135.862) (angle 90) (layer Edge.Cuts) (width 0.1524))
 (gr_line (start 104.842 139.662) (end 112.942 139.662) (layer Edge.Cuts) (width 0.1524))
 (gr_arc (start 104.842 135.862) (end 104.842 139.662) (angle 90) (layer Edge.Cuts) (width 0.1524))
 (gr_line (start 116.146 87.162) (end 100.546 87.162) (layer Edge.Cuts) (width 0.1524))
 (gr_line (start 96.546 67.562) (end 96.546 83.462) (layer Edge.Cuts) (width 0.1524))
 (gr_arc (start 100.541009 83.16225) (end 100.541009 87.16225) (angle 87.13760121) (layer Edge.Cuts) (width 0.1524))
 (gr_arc (start 100.546 67.562) (end 96.546 67.562) (angle 90) (layer Edge.Cuts) (width 0.1524))
 (gr_line (start 116.146 63.562) (end 100.346 63.562) (layer Edge.Cuts) (width 0.1524))
 (gr_arc (start 116.146 83.162) (end 120.146 83.162) (angle 90) (layer Edge.Cuts) (width 0.1524))
 (gr_line (start 120.146 83.162) (end 120.146 67.262) (layer Edge.Cuts) (width 0.1524))
 (gr_arc (start 116.150991 67.56175) (end 116.150991 63.56175) (angle 87.13760121) (layer Edge.Cuts) (width 0.1524))
 (gr_line (start 90.038 87.216) (end 66.138 87.216) (layer Edge.Cuts) (width 0.1524))
 (gr_line (start 66.138 63.616) (end 90.138 63.616) (layer Edge.Cuts) (width 0.1524))
 (gr_line (start 93.938 83.216) (end 93.938 67.316) (layer Edge.Cuts) (width 0.1524))
 (gr_arc (start 89.942991 67.61575) (end 89.942991 63.61575) (angle 87.13760121) (layer Edge.Cuts) (width 0.1524))
 (gr_arc (start 89.938 83.216) (end 93.938 83.216) (angle 90) (layer Edge.Cuts) (width 0.1524))
 (gr_line (start 62.238 67.616) (end 62.238 83.516) (layer Edge.Cuts) (width 0.1524))
 (gr_arc (start 66.233009 83.21625) (end 66.233009 87.21625) (angle 87.13760121) (layer Edge.Cuts) (width 0.1524))
 (gr_arc (start 66.238 67.616) (end 62.238 67.616) (angle 90) (layer Edge.Cuts) (width 0.1524))
 (gr_line (start 118.746 93.47) (end 118.746 117.57) (layer Edge.Cuts) (width 0.1524))
 (gr_arc (start 114.752159 93.67) (end 114.752159 89.67) (angle 86.82016988) (layer Edge.Cuts) (width 0.1524))
 (gr_line (start 66.546 89.77) (end 115.082 89.682) (layer Edge.Cuts) (width 0.1524))
 (gr_arc (start 66.546 93.37) (end 62.946 93.37) (angle 90) (layer Edge.Cuts) (width 0.1524))
 (gr_line (start 62.946 117.67) (end 62.946 93.27) (layer Edge.Cuts) (width 0.1524))
 (gr_arc (start 66.746 117.67) (end 66.746 121.47) (angle 90) (layer Edge.Cuts) (width 0.1524))
 (gr_line (start 114.946 121.47) (end 66.646 121.47) (layer Edge.Cuts) (width 0.1524))
 (gr_arc (start 114.846 117.57) (end 118.746 117.57) (angle 88.49256424) (layer Edge.Cuts) (width 0.1524))
 (segment (start 102.807 106.971) (end 102.807 94.331) (width 0.508) (layer F.Cu) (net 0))
 (segment (start 97.046 110.77) (end 108.006 110.77) (width 0.254) (layer F.Cu) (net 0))
 (segment (start 108.006 110.77) (end 114.826 117.59) (width 0.254) (layer F.Cu) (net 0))
 (segment (start 96.546 110.27) (end 97.046 110.77) (width 0.254) (layer F.Cu) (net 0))
 (segment (start 96.446 110.27) (end 96.546 110.27) (width 0.254) (layer F.Cu) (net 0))
 (segment (start 97.727 106.971) (end 97.727 108.192314) (width 0.254) (layer F.Cu) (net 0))
 (segment (start 97.727 108.192314) (end 99.125686 109.591) (width 0.254) (layer F.Cu) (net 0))
 (segment (start 99.125686 109.591) (end 114.826 109.591) (width 0.254) (layer F.Cu) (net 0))
 (segment (start 95.187 109.011) (end 96.446 110.27) (width 0.254) (layer F.Cu) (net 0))
 (segment (start 95.187 106.971) (end 95.187 109.011) (width 0.254) (layer F.Cu) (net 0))
 (segment (start 95.746 111.77) (end 101.006 111.77) (width 0.254) (layer F.Cu) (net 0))
 (segment (start 101.006 111.77) (end 106.826 117.59) (width 0.254) (layer F.Cu) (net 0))
 (segment (start 92.647 108.671) (end 95.746 111.77) (width 0.254) (layer F.Cu) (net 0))
 (segment (start 92.647 106.971) (end 92.647 108.671) (width 0.254) (layer F.Cu) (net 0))
 (segment (start 90.107 106.971) (end 90.107 108.871) (width 0.254) (layer F.Cu) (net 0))
 (segment (start 90.107 108.871) (end 98.826 117.59) (width 0.254) (layer F.Cu) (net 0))
 (segment (start 87.567 106.971) (end 87.567 114.331) (width 0.254) (layer F.Cu) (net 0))
 (segment (start 87.567 114.331) (end 90.826 117.59) (width 0.254) (layer F.Cu) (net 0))
 (segment (start 85.027 106.971) (end 85.027 115.389) (width 0.254) (layer F.Cu) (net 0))
 (segment (start 85.027 115.389) (end 82.826 117.59) (width 0.254) (layer F.Cu) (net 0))
 (segment (start 82.487 106.971) (end 82.487 109.93) (width 0.254) (layer F.Cu) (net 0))
 (segment (start 82.487 109.93) (end 74.826 117.591) (width 0.254) (layer F.Cu) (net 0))
 (segment (start 79.947 106.971) (end 74.848 112.07) (width 0.254) (layer F.Cu) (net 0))
 (segment (start 74.848 112.07) (end 72.346 112.07) (width 0.254) (layer F.Cu) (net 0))
 (segment (start 72.346 112.07) (end 66.826 117.59) (width 0.254) (layer F.Cu) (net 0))
 (segment (start 66.826 109.591) (end 74.787 109.591) (width 0.254) (layer F.Cu) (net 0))
 (segment (start 74.787 109.591) (end 77.407 106.971) (width 0.254) (layer F.Cu) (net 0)))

